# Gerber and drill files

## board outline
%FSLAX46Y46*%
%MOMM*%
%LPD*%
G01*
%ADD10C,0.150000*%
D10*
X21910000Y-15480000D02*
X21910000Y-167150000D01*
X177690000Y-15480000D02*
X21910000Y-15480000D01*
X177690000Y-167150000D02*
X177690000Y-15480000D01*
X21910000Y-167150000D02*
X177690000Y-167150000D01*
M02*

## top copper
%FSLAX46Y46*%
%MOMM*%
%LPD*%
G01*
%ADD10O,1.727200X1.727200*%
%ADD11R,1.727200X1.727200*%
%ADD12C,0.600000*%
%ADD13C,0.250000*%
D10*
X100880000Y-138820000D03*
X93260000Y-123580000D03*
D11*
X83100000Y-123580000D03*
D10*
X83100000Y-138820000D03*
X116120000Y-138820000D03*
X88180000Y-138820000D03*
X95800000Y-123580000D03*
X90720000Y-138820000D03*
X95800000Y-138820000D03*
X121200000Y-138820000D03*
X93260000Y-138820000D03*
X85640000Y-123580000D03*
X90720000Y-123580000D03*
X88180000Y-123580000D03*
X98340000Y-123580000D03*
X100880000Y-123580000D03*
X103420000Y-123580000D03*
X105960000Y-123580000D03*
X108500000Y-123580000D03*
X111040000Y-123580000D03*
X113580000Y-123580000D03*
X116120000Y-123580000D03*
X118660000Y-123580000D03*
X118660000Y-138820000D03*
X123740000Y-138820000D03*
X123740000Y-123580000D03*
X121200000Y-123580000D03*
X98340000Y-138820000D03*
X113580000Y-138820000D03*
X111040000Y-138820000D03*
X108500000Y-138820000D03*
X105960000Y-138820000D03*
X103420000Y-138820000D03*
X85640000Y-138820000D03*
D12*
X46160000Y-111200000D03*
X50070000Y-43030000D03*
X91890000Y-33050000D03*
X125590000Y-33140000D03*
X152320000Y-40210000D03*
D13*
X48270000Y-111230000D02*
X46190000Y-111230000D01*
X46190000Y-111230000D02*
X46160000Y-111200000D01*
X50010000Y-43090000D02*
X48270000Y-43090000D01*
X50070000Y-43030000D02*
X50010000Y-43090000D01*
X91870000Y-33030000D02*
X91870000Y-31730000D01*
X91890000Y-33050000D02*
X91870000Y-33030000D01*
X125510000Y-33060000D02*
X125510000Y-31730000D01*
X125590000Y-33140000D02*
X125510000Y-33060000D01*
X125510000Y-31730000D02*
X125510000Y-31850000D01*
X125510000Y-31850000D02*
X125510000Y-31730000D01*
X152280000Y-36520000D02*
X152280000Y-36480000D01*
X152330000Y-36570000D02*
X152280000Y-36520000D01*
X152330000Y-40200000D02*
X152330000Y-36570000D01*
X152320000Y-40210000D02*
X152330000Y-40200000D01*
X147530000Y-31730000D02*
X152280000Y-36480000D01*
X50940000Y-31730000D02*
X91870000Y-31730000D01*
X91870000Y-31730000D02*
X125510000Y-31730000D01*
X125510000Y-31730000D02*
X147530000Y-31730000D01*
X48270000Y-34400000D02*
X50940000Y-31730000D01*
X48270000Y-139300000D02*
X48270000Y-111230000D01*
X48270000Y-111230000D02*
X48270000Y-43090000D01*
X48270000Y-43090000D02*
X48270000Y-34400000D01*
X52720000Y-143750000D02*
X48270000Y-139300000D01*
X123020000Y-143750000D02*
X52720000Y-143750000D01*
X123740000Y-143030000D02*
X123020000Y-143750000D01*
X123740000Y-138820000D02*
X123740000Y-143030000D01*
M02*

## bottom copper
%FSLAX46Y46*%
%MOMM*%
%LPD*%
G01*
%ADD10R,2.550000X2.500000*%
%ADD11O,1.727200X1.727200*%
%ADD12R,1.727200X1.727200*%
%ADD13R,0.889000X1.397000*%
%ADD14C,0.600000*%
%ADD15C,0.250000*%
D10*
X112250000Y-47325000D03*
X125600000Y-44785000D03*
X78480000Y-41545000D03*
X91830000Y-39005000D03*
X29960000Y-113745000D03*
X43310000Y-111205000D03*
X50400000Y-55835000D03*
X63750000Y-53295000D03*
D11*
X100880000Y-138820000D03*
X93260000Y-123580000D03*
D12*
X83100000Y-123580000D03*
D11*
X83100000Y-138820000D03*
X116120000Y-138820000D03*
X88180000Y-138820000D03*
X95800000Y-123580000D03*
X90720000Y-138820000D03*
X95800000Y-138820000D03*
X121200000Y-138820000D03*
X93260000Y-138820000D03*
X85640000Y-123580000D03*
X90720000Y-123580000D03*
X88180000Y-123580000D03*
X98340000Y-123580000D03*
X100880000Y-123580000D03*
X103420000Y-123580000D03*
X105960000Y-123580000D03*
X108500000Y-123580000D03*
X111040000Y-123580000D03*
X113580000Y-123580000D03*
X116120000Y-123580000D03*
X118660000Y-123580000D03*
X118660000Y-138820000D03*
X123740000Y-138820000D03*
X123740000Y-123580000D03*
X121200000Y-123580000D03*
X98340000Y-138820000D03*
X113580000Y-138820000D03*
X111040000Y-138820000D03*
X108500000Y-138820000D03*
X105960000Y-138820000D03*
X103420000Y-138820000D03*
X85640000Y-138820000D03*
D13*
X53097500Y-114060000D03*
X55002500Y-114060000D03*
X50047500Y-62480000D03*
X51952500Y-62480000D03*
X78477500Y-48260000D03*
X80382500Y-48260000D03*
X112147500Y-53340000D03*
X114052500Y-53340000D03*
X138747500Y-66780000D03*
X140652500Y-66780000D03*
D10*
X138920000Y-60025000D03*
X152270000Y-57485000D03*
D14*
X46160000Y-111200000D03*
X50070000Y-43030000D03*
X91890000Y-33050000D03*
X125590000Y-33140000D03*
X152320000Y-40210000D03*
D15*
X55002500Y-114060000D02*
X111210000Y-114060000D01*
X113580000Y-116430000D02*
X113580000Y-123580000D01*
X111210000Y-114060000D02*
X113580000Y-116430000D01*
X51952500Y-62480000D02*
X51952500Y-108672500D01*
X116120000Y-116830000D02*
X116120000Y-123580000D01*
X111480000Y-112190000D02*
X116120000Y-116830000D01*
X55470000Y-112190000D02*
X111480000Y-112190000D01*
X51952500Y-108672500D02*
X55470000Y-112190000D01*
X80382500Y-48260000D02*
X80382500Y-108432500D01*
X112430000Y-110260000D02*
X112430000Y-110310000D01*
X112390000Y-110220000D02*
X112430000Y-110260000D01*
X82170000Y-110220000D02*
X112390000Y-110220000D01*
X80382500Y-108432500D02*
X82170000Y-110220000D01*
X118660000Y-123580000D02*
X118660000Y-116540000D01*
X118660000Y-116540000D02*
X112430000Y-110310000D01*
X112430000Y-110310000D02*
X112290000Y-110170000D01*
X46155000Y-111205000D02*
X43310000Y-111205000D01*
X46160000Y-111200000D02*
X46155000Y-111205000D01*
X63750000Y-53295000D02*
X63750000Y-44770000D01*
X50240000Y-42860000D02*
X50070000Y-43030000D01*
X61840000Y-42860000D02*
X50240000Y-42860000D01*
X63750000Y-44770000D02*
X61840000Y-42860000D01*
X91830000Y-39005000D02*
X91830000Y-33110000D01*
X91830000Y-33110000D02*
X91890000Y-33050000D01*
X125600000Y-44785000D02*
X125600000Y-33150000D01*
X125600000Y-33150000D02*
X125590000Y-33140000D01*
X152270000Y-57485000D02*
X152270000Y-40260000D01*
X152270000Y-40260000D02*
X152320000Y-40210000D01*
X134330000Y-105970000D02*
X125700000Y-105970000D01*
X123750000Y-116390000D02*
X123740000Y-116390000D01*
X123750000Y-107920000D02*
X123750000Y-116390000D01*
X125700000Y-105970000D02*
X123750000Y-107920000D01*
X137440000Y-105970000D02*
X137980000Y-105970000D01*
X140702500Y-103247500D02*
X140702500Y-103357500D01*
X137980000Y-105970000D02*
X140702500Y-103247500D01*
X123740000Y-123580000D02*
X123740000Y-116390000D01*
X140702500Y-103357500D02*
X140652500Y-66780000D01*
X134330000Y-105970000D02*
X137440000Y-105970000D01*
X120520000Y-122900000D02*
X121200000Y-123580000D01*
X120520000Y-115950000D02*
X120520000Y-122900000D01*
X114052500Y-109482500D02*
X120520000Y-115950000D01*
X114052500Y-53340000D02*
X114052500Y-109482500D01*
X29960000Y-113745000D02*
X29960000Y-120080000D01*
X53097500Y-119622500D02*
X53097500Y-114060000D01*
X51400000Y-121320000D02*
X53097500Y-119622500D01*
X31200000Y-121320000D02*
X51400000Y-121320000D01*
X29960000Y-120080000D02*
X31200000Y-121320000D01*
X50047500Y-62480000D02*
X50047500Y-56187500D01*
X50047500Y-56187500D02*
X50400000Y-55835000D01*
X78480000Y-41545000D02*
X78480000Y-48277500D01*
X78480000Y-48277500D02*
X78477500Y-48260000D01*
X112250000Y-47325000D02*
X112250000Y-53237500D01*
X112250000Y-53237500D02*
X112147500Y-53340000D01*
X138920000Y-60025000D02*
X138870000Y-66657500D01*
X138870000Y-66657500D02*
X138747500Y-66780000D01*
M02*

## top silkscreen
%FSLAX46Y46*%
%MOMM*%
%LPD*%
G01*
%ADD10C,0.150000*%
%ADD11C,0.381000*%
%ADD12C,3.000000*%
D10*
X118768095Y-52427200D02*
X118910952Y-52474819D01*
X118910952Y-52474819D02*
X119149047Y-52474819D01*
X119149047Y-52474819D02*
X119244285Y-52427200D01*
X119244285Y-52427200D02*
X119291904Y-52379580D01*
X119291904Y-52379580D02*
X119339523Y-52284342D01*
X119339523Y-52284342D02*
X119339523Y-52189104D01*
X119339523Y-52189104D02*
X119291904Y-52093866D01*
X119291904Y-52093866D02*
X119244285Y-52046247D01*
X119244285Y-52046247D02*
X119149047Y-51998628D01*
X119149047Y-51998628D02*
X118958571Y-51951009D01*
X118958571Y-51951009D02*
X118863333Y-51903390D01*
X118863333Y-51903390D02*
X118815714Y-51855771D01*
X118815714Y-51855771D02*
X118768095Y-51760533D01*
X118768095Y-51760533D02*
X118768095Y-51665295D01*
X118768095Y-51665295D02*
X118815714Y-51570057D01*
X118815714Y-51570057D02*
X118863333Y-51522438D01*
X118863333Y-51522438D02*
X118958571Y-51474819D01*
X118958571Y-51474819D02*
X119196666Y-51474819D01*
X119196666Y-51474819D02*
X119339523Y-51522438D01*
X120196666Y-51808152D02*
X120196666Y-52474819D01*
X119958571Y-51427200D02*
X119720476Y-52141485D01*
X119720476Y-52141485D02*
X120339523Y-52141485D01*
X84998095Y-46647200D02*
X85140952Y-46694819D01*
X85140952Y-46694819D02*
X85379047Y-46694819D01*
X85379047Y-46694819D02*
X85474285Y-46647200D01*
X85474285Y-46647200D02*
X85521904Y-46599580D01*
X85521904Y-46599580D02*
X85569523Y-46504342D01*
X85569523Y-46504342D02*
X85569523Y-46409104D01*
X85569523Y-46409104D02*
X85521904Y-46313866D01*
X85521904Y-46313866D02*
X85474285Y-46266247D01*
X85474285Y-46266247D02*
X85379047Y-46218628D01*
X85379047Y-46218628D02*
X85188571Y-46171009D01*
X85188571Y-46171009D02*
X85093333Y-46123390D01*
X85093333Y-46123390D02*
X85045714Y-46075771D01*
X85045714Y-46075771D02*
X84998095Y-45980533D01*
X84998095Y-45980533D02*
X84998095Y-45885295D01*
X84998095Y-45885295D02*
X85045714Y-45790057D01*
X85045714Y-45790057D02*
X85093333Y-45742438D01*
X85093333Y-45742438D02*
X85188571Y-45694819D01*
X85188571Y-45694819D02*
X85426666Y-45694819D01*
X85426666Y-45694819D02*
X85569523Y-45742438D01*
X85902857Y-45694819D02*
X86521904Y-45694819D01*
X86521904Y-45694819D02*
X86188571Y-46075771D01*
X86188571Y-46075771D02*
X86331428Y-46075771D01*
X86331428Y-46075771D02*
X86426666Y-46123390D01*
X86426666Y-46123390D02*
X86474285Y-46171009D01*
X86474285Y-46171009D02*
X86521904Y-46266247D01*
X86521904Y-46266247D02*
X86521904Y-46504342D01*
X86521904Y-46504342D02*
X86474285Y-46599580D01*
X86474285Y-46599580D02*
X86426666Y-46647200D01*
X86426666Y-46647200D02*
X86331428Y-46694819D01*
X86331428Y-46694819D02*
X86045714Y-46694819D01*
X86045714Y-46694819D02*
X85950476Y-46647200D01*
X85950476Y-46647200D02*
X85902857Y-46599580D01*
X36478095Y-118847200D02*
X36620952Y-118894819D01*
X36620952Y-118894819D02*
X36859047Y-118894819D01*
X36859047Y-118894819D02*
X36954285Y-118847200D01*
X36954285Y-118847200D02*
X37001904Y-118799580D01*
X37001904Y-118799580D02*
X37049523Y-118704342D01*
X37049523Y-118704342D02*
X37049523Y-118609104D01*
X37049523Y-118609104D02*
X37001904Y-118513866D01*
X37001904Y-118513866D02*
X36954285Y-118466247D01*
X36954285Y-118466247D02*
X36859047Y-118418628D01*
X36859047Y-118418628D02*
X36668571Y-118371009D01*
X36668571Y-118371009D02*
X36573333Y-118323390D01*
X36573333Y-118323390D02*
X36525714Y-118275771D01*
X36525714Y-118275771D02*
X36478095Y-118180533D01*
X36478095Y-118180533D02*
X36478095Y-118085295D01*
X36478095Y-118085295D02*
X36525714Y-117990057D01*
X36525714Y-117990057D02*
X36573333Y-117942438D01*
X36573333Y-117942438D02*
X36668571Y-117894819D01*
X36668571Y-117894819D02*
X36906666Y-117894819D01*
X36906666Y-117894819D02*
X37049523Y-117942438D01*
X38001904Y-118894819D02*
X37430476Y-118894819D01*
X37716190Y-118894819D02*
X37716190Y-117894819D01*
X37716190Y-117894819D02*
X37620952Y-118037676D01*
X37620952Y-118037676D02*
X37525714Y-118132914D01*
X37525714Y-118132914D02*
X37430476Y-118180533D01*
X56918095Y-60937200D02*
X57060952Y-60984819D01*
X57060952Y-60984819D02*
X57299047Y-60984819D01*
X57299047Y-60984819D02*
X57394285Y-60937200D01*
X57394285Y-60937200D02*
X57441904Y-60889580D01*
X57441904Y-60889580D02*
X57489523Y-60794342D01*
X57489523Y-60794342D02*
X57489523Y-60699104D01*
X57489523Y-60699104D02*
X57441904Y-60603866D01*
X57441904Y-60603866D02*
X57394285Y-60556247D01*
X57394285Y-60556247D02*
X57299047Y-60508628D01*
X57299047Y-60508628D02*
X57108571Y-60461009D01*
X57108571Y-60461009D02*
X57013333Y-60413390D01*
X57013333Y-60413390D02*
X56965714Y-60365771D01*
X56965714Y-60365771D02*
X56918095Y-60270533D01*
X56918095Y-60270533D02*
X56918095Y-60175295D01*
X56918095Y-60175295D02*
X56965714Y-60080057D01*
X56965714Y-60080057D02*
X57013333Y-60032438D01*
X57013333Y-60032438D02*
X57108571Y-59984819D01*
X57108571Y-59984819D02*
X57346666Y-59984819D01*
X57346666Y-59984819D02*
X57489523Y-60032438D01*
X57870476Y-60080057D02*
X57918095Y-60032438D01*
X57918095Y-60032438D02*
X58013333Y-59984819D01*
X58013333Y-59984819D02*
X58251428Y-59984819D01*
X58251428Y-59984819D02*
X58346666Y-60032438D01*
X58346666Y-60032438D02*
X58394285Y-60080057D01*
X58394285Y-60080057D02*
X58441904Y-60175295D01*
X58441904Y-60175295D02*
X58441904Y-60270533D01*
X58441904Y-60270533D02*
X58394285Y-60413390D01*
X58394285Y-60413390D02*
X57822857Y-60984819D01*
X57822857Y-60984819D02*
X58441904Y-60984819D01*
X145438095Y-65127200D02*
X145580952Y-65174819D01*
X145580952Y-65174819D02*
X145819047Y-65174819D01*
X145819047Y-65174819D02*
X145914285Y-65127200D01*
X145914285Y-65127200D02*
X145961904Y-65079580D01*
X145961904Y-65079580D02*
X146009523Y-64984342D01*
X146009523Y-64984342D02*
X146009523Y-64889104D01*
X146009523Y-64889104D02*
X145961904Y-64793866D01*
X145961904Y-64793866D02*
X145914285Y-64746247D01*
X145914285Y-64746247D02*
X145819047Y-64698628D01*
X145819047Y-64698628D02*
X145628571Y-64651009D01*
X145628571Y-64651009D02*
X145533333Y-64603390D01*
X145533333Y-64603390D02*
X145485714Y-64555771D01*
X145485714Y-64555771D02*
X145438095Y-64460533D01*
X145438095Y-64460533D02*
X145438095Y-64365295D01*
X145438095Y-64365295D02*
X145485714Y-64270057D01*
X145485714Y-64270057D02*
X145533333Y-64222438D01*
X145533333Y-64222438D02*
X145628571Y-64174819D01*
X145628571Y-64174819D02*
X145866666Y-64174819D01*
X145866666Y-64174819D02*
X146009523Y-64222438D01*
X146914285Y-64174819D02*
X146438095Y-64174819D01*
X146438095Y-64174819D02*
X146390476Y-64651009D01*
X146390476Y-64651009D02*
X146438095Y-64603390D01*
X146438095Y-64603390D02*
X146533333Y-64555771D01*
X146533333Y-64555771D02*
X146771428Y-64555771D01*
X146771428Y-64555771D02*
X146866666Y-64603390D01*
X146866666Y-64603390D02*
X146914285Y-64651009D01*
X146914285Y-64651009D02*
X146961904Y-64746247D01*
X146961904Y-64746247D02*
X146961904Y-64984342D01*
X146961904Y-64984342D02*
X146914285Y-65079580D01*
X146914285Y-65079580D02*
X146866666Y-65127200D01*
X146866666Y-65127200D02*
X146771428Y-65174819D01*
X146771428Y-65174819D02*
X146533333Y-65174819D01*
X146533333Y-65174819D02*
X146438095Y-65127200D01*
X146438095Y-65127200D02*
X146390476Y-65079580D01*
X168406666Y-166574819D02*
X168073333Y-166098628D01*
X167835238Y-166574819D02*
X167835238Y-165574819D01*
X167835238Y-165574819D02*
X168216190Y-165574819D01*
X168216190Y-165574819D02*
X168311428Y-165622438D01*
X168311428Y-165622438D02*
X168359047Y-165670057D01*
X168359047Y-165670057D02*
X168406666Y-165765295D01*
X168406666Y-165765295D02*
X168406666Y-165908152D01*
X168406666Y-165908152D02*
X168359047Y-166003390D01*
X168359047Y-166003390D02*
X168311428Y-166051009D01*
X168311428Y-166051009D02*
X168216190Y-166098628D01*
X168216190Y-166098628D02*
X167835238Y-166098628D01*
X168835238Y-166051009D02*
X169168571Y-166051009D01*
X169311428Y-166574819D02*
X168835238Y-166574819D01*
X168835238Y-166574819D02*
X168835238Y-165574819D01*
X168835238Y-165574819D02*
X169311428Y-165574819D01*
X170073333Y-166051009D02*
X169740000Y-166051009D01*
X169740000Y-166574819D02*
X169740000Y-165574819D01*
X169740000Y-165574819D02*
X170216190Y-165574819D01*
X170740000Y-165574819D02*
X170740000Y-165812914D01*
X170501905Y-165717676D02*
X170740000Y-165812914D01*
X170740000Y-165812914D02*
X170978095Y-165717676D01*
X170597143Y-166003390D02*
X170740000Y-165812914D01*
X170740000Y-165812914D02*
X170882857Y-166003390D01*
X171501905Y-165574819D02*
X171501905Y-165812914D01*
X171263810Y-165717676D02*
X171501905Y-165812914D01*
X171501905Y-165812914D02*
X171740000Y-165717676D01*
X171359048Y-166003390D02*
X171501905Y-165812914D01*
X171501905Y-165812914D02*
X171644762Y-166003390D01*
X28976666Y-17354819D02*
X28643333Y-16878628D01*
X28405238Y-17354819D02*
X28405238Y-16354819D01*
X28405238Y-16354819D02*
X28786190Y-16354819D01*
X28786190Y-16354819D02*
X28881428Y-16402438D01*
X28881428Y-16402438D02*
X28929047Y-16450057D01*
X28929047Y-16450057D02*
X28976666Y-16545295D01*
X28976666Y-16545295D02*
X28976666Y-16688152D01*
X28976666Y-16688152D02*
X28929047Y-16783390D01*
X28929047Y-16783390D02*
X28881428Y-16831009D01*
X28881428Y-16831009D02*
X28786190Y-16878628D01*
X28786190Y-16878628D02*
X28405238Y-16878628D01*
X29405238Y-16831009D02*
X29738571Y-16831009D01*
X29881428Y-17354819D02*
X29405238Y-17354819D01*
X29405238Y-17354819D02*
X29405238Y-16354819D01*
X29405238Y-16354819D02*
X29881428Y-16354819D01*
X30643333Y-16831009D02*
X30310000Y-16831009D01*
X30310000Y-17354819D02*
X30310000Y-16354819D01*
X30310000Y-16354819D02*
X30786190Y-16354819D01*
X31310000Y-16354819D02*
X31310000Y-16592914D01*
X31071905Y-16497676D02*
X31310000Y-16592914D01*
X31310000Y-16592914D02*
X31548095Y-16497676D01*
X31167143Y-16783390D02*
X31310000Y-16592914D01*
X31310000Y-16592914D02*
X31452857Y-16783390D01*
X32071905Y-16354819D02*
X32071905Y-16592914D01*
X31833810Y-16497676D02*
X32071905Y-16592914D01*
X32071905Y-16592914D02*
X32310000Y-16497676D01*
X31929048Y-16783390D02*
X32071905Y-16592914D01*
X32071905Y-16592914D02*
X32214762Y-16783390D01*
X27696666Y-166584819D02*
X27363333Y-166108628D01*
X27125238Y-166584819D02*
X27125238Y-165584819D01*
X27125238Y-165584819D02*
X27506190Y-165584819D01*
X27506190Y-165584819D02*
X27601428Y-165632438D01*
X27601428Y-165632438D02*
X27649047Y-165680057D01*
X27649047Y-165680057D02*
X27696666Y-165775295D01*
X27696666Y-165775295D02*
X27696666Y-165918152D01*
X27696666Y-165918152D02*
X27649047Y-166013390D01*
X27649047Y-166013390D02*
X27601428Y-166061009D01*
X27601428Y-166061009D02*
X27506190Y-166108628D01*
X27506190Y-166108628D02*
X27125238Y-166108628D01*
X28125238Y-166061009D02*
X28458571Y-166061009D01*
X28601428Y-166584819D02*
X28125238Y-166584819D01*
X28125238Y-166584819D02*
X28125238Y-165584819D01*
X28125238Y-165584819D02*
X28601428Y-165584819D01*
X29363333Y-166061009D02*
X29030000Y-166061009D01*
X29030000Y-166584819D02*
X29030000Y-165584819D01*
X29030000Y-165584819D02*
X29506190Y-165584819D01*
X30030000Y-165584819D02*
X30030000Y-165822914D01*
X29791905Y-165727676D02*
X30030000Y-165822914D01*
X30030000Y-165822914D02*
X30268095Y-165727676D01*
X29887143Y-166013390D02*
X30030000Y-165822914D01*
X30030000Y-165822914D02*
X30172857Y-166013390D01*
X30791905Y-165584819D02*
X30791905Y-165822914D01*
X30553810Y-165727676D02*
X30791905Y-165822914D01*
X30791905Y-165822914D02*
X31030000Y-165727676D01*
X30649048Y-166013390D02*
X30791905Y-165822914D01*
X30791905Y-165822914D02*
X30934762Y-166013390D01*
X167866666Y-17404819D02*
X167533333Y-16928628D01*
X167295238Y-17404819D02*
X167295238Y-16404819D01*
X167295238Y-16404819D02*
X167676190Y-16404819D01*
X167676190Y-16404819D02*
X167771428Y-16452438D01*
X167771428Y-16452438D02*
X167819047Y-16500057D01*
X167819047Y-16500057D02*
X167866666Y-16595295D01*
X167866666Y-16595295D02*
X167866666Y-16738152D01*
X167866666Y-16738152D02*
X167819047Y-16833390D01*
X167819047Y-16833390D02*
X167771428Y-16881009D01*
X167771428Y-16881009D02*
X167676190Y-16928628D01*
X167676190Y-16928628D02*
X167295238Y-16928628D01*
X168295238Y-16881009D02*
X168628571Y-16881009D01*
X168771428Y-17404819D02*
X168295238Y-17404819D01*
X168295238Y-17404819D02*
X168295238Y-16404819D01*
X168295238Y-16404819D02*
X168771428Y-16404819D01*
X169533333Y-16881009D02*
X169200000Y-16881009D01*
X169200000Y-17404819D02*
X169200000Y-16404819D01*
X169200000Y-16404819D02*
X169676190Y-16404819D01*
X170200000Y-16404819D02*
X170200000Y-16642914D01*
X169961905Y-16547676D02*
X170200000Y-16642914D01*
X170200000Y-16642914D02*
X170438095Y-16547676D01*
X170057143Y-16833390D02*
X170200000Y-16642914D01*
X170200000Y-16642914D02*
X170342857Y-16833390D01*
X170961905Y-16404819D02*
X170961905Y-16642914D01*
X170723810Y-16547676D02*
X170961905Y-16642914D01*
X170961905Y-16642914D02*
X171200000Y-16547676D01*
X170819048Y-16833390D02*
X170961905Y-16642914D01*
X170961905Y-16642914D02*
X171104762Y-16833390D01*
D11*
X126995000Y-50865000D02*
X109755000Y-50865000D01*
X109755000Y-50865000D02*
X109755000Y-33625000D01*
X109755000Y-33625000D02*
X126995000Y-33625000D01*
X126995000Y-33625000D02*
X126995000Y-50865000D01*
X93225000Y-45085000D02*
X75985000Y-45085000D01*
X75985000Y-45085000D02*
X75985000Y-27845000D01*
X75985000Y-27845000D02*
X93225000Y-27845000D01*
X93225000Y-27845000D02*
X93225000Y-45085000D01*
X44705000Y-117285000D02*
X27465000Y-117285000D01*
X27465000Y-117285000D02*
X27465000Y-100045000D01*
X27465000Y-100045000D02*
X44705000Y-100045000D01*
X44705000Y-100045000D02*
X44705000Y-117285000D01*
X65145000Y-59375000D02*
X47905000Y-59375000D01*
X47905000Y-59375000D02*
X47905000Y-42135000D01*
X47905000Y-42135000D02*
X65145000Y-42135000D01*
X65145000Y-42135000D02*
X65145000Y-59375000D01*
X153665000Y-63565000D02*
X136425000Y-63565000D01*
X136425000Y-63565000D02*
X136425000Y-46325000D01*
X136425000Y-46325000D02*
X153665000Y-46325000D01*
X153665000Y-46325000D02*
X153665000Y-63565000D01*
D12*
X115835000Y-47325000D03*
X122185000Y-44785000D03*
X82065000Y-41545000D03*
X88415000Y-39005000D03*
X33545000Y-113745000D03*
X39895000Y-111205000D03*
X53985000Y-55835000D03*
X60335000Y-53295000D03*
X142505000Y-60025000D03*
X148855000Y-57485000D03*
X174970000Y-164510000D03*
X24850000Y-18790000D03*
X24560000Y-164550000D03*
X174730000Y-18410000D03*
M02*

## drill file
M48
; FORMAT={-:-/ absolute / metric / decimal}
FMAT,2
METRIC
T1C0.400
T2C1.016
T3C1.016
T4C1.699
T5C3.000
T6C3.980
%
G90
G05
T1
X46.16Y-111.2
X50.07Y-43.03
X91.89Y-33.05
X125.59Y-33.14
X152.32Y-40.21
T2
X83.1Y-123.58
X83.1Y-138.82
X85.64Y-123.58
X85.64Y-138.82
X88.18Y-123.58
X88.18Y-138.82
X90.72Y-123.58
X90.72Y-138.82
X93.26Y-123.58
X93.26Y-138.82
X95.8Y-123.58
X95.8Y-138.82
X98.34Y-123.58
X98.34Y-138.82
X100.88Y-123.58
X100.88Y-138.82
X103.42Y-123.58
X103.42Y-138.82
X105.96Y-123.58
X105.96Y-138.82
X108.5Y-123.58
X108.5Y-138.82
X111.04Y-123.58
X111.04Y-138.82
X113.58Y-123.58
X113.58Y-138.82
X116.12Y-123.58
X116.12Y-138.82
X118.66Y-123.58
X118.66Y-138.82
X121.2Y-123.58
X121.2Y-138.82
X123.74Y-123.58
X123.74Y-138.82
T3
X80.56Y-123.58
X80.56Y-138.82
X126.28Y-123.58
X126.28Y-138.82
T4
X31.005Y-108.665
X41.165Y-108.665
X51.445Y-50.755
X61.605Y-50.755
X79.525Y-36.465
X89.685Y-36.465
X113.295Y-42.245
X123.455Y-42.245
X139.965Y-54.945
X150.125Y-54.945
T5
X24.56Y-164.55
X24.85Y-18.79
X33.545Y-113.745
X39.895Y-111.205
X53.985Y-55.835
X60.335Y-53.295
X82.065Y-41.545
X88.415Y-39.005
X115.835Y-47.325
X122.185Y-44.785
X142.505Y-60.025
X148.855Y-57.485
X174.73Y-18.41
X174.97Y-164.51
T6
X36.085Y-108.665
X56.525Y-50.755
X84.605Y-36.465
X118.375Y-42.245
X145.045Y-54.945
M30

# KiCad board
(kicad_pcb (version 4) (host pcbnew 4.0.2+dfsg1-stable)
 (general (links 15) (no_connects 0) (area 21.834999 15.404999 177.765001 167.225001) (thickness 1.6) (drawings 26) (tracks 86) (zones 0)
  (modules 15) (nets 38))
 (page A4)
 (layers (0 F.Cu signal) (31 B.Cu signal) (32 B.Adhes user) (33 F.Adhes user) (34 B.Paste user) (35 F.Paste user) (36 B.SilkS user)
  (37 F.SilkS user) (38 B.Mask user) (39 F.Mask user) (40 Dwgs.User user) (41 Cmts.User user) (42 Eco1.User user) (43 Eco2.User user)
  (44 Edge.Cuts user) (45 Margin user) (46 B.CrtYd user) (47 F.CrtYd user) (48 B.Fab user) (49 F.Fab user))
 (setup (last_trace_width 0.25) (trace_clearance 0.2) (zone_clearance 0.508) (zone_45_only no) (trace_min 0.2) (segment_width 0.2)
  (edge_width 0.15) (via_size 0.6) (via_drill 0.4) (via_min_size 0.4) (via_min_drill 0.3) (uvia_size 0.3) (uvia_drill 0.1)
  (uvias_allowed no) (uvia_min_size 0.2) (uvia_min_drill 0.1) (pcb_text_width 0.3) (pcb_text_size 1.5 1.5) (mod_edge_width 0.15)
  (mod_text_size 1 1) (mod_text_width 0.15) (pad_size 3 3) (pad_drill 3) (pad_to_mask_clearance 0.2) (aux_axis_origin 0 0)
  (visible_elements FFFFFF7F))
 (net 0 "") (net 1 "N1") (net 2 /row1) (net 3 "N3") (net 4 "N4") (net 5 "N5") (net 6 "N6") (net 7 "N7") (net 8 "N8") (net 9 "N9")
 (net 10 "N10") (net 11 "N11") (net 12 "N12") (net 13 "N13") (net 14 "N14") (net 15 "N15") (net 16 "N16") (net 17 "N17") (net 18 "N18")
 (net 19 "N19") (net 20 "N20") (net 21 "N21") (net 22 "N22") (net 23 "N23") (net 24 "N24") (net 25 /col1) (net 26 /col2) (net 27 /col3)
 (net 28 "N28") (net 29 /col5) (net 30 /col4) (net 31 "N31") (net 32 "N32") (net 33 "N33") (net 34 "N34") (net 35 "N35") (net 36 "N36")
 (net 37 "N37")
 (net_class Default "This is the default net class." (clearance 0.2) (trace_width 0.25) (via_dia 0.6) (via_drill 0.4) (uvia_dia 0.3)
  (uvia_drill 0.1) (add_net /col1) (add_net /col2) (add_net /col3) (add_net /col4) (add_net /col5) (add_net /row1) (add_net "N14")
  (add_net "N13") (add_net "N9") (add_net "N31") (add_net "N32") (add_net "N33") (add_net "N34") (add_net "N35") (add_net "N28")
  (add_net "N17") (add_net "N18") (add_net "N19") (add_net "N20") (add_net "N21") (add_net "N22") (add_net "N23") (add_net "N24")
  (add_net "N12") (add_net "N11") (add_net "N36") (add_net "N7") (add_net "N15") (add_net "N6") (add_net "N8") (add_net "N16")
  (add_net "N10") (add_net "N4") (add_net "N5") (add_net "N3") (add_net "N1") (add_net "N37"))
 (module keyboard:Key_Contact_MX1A (layer F.Cu) (at 118.43 42.29)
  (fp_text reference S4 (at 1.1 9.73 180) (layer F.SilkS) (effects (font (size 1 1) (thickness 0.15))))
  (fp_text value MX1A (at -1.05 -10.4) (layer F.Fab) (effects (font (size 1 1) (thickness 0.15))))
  (fp_line (start 8.565 8.575) (end -8.675 8.575) (layer F.SilkS) (width 0.381))
  (fp_line (start -8.675 8.575) (end -8.675 -8.665) (layer F.SilkS) (width 0.381))
  (fp_line (start -8.675 -8.665) (end 8.565 -8.665) (layer F.SilkS) (width 0.381))
  (fp_line (start 8.565 -8.665) (end 8.565 8.575) (layer F.SilkS) (width 0.381))
  (pad "" np_thru_hole circle (at -0.055 -0.045 180) (size 3.98018 3.98018) (drill 3.98018) (layers *.Cu *.Mask))
  (pad "" np_thru_hole circle (at -2.595 5.035 180) (size 3 3) (drill 3) (layers *.Cu *.Mask F.SilkS))
  (pad "" np_thru_hole circle (at 3.755 2.495 180) (size 3 3) (drill 3) (layers *.Cu *.Mask F.SilkS))
  (pad "" np_thru_hole circle (at 5.025 -0.045 180) (size 1.69926 1.69926) (drill 1.69926) (layers *.Cu *.Mask))
  (pad "" np_thru_hole circle (at -5.135 -0.045 180) (size 1.69926 1.69926) (drill 1.69926) (layers *.Cu *.Mask))
  (pad 2 smd rect (at -6.18 5.035) (size 2.55 2.5) (layers B.Cu B.Paste B.Mask) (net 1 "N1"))
  (pad 1 smd rect (at 7.17 2.495 180) (size 2.55 2.5) (layers B.Cu B.Paste B.Mask) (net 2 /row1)))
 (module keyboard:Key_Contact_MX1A (layer F.Cu) (at 84.66 36.51)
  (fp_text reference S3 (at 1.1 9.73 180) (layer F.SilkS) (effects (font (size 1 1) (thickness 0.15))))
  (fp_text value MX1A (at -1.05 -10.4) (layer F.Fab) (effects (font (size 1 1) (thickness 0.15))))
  (fp_line (start 8.565 8.575) (end -8.675 8.575) (layer F.SilkS) (width 0.381))
  (fp_line (start -8.675 8.575) (end -8.675 -8.665) (layer F.SilkS) (width 0.381))
  (fp_line (start -8.675 -8.665) (end 8.565 -8.665) (layer F.SilkS) (width 0.381))
  (fp_line (start 8.565 -8.665) (end 8.565 8.575) (layer F.SilkS) (width 0.381))
  (pad "" np_thru_hole circle (at -0.055 -0.045 180) (size 3.98018 3.98018) (drill 3.98018) (layers *.Cu *.Mask))
  (pad "" np_thru_hole circle (at -2.595 5.035 180) (size 3 3) (drill 3) (layers *.Cu *.Mask F.SilkS))
  (pad "" np_thru_hole circle (at 3.755 2.495 180) (size 3 3) (drill 3) (layers *.Cu *.Mask F.SilkS))
  (pad "" np_thru_hole circle (at 5.025 -0.045 180) (size 1.69926 1.69926) (drill 1.69926) (layers *.Cu *.Mask))
  (pad "" np_thru_hole circle (at -5.135 -0.045 180) (size 1.69926 1.69926) (drill 1.69926) (layers *.Cu *.Mask))
  (pad 2 smd rect (at -6.18 5.035) (size 2.55 2.5) (layers B.Cu B.Paste B.Mask) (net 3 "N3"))
  (pad 1 smd rect (at 7.17 2.495 180) (size 2.55 2.5) (layers B.Cu B.Paste B.Mask) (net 2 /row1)))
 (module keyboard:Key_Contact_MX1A (layer F.Cu) (at 36.14 108.71)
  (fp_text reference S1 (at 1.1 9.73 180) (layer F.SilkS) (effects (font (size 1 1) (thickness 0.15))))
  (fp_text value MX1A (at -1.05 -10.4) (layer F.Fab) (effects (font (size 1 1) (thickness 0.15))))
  (fp_line (start 8.565 8.575) (end -8.675 8.575) (layer F.SilkS) (width 0.381))
  (fp_line (start -8.675 8.575) (end -8.675 -8.665) (layer F.SilkS) (width 0.381))
  (fp_line (start -8.675 -8.665) (end 8.565 -8.665) (layer F.SilkS) (width 0.381))
  (fp_line (start 8.565 -8.665) (end 8.565 8.575) (layer F.SilkS) (width 0.381))
  (pad "" np_thru_hole circle (at -0.055 -0.045 180) (size 3.98018 3.98018) (drill 3.98018) (layers *.Cu *.Mask))
  (pad "" np_thru_hole circle (at -2.595 5.035 180) (size 3 3) (drill 3) (layers *.Cu *.Mask F.SilkS))
  (pad "" np_thru_hole circle (at 3.755 2.495 180) (size 3 3) (drill 3) (layers *.Cu *.Mask F.SilkS))
  (pad "" np_thru_hole circle (at 5.025 -0.045 180) (size 1.69926 1.69926) (drill 1.69926) (layers *.Cu *.Mask))
  (pad "" np_thru_hole circle (at -5.135 -0.045 180) (size 1.69926 1.69926) (drill 1.69926) (layers *.Cu *.Mask))
  (pad 2 smd rect (at -6.18 5.035) (size 2.55 2.5) (layers B.Cu B.Paste B.Mask) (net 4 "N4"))
  (pad 1 smd rect (at 7.17 2.495 180) (size 2.55 2.5) (layers B.Cu B.Paste B.Mask) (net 2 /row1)))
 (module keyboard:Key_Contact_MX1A (layer F.Cu) (at 56.58 50.8)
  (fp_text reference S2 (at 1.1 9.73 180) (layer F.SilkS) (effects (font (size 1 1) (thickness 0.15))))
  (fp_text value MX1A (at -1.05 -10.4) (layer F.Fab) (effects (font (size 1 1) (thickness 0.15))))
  (fp_line (start 8.565 8.575) (end -8.675 8.575) (layer F.SilkS) (width 0.381))
  (fp_line (start -8.675 8.575) (end -8.675 -8.665) (layer F.SilkS) (width 0.381))
  (fp_line (start -8.675 -8.665) (end 8.565 -8.665) (layer F.SilkS) (width 0.381))
  (fp_line (start 8.565 -8.665) (end 8.565 8.575) (layer F.SilkS) (width 0.381))
  (pad "" np_thru_hole circle (at -0.055 -0.045 180) (size 3.98018 3.98018) (drill 3.98018) (layers *.Cu *.Mask))
  (pad "" np_thru_hole circle (at -2.595 5.035 180) (size 3 3) (drill 3) (layers *.Cu *.Mask F.SilkS))
  (pad "" np_thru_hole circle (at 3.755 2.495 180) (size 3 3) (drill 3) (layers *.Cu *.Mask F.SilkS))
  (pad "" np_thru_hole circle (at 5.025 -0.045 180) (size 1.69926 1.69926) (drill 1.69926) (layers *.Cu *.Mask))
  (pad "" np_thru_hole circle (at -5.135 -0.045 180) (size 1.69926 1.69926) (drill 1.69926) (layers *.Cu *.Mask))
  (pad 2 smd rect (at -6.18 5.035) (size 2.55 2.5) (layers B.Cu B.Paste B.Mask) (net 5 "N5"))
  (pad 1 smd rect (at 7.17 2.495 180) (size 2.55 2.5) (layers B.Cu B.Paste B.Mask) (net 2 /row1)))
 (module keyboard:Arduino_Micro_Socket (layer B.Cu) (at 127.66 140.2 180)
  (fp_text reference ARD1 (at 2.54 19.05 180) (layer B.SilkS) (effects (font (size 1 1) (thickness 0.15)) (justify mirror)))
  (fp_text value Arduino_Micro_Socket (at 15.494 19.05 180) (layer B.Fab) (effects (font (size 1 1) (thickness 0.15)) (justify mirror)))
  (pad "" np_thru_hole circle (at 47.1 16.62 180) (size 1.016 1.016) (drill 1.016) (layers *.Cu *.Mask))
  (pad "" np_thru_hole circle (at 1.38 16.62 180) (size 1.016 1.016) (drill 1.016) (layers *.Cu *.Mask))
  (pad "" np_thru_hole circle (at 47.1 1.38 180) (size 1.016 1.016) (drill 1.016) (layers *.Cu *.Mask))
  (pad "" thru_hole oval (at 26.78 1.38 180) (size 1.7272 1.7272) (drill 1.016) (layers *.Cu *.Mask))
  (pad RST2 thru_hole oval (at 34.4 16.62 180) (size 1.7272 1.7272) (drill 1.016) (layers *.Cu *.Mask) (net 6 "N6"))
  (pad MOSI thru_hole rect (at 44.56 16.62 180) (size 1.7272 1.7272) (drill 1.016) (layers *.Cu *.Mask) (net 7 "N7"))
  (pad SCK thru_hole oval (at 44.56 1.38 180) (size 1.7272 1.7272) (drill 1.016) (layers *.Cu *.Mask) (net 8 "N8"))
  (pad A0 thru_hole oval (at 11.54 1.38 180) (size 1.7272 1.7272) (drill 1.016) (layers *.Cu *.Mask) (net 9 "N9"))
  (pad VIN thru_hole oval (at 39.48 1.38 180) (size 1.7272 1.7272) (drill 1.016) (layers *.Cu *.Mask) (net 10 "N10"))
  (pad GND2 thru_hole oval (at 31.86 16.62 180) (size 1.7272 1.7272) (drill 1.016) (layers *.Cu *.Mask) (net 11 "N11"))
  (pad GND1 thru_hole oval (at 36.94 1.38 180) (size 1.7272 1.7272) (drill 1.016) (layers *.Cu *.Mask) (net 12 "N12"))
  (pad 5V thru_hole oval (at 31.86 1.38 180) (size 1.7272 1.7272) (drill 1.016) (layers *.Cu *.Mask) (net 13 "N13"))
  (pad 3.3V thru_hole oval (at 6.46 1.38 180) (size 1.7272 1.7272) (drill 1.016) (layers *.Cu *.Mask) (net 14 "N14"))
  (pad RST1 thru_hole oval (at 34.4 1.38 180) (size 1.7272 1.7272) (drill 1.016) (layers *.Cu *.Mask) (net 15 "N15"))
  (pad SS thru_hole oval (at 42.02 16.62 180) (size 1.7272 1.7272) (drill 1.016) (layers *.Cu *.Mask) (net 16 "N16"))
  (pad D0 thru_hole oval (at 36.94 16.62 180) (size 1.7272 1.7272) (drill 1.016) (layers *.Cu *.Mask) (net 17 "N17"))
  (pad D1 thru_hole oval (at 39.48 16.62 180) (size 1.7272 1.7272) (drill 1.016) (layers *.Cu *.Mask) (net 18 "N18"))
  (pad D2 thru_hole oval (at 29.32 16.62 180) (size 1.7272 1.7272) (drill 1.016) (layers *.Cu *.Mask) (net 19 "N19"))
  (pad D3 thru_hole oval (at 26.78 16.62 180) (size 1.7272 1.7272) (drill 1.016) (layers *.Cu *.Mask) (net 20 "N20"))
  (pad D4 thru_hole oval (at 24.24 16.62 180) (size 1.7272 1.7272) (drill 1.016) (layers *.Cu *.Mask) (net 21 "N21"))
  (pad D5 thru_hole oval (at 21.7 16.62 180) (size 1.7272 1.7272) (drill 1.016) (layers *.Cu *.Mask) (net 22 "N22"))
  (pad D6 thru_hole oval (at 19.16 16.62 180) (size 1.7272 1.7272) (drill 1.016) (layers *.Cu *.Mask) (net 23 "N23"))
  (pad D7 thru_hole oval (at 16.62 16.62 180) (size 1.7272 1.7272) (drill 1.016) (layers *.Cu *.Mask) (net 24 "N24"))
  (pad D8 thru_hole oval (at 14.08 16.62 180) (size 1.7272 1.7272) (drill 1.016) (layers *.Cu *.Mask) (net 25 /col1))
  (pad D9 thru_hole oval (at 11.54 16.62 180) (size 1.7272 1.7272) (drill 1.016) (layers *.Cu *.Mask) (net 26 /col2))
  (pad D10 thru_hole oval (at 9 16.62 180) (size 1.7272 1.7272) (drill 1.016) (layers *.Cu *.Mask) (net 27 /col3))
  (pad "" np_thru_hole circle (at 1.38 1.38 180) (size 1.016 1.016) (drill 1.016) (layers *.Cu *.Mask))
  (pad AREF thru_hole oval (at 9 1.38 180) (size 1.7272 1.7272) (drill 1.016) (layers *.Cu *.Mask) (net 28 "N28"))
  (pad D13 thru_hole oval (at 3.92 1.38 180) (size 1.7272 1.7272) (drill 1.016) (layers *.Cu *.Mask) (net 2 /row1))
  (pad D12 thru_hole oval (at 3.92 16.62 180) (size 1.7272 1.7272) (drill 1.016) (layers *.Cu *.Mask) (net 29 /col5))
  (pad D11 thru_hole oval (at 6.46 16.62 180) (size 1.7272 1.7272) (drill 1.016) (layers *.Cu *.Mask) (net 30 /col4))
  (pad "" thru_hole oval (at 29.32 1.38 180) (size 1.7272 1.7272) (drill 1.016) (layers *.Cu *.Mask))
  (pad A1 thru_hole oval (at 14.08 1.38 180) (size 1.7272 1.7272) (drill 1.016) (layers *.Cu *.Mask) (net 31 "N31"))
  (pad A2 thru_hole oval (at 16.62 1.38 180) (size 1.7272 1.7272) (drill 1.016) (layers *.Cu *.Mask) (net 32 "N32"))
  (pad A3 thru_hole oval (at 19.16 1.38 180) (size 1.7272 1.7272) (drill 1.016) (layers *.Cu *.Mask) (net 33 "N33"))
  (pad A4 thru_hole oval (at 21.7 1.38 180) (size 1.7272 1.7272) (drill 1.016) (layers *.Cu *.Mask) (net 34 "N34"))
  (pad A5 thru_hole oval (at 24.24 1.38 180) (size 1.7272 1.7272) (drill 1.016) (layers *.Cu *.Mask) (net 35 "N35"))
  (pad MISO thru_hole oval (at 42.02 1.38 180) (size 1.7272 1.7272) (drill 1.016) (layers *.Cu *.Mask) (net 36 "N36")))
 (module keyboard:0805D (layer B.Cu) (at 54.05 114.06)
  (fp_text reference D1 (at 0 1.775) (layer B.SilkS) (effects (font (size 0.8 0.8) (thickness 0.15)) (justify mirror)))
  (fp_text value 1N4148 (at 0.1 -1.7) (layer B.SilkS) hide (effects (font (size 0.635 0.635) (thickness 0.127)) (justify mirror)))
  (pad 1 smd rect (at -0.9525 0) (size 0.889 1.397) (layers B.Cu B.Paste B.Mask) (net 4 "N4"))
  (pad 2 smd rect (at 0.9525 0) (size 0.889 1.397) (layers B.Cu B.Paste B.Mask) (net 25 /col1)))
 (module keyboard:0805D (layer B.Cu) (at 51 62.48)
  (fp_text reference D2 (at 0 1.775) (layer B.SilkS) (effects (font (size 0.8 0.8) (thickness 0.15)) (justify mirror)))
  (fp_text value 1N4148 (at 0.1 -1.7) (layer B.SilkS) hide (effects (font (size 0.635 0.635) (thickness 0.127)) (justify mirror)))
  (pad 1 smd rect (at -0.9525 0) (size 0.889 1.397) (layers B.Cu B.Paste B.Mask) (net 5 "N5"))
  (pad 2 smd rect (at 0.9525 0) (size 0.889 1.397) (layers B.Cu B.Paste B.Mask) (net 26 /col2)))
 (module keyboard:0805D (layer B.Cu) (at 79.43 48.26)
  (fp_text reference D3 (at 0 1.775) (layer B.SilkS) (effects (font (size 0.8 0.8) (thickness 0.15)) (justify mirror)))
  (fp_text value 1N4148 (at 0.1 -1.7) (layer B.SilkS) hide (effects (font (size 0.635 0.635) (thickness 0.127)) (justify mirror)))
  (pad 1 smd rect (at -0.9525 0) (size 0.889 1.397) (layers B.Cu B.Paste B.Mask) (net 3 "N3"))
  (pad 2 smd rect (at 0.9525 0) (size 0.889 1.397) (layers B.Cu B.Paste B.Mask) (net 27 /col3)))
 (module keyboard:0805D (layer B.Cu) (at 113.1 53.34)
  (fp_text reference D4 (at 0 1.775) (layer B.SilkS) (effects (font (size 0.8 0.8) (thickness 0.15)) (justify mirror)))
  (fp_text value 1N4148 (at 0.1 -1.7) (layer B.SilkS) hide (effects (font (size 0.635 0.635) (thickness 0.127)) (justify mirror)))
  (pad 1 smd rect (at -0.9525 0) (size 0.889 1.397) (layers B.Cu B.Paste B.Mask) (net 1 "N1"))
  (pad 2 smd rect (at 0.9525 0) (size 0.889 1.397) (layers B.Cu B.Paste B.Mask) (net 30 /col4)))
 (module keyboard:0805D (layer B.Cu) (at 139.7 66.78)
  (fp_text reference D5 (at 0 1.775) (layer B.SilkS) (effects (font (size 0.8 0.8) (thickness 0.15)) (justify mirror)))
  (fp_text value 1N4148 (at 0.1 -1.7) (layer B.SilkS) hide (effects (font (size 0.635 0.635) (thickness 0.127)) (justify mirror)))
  (pad 1 smd rect (at -0.9525 0) (size 0.889 1.397) (layers B.Cu B.Paste B.Mask) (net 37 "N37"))
  (pad 2 smd rect (at 0.9525 0) (size 0.889 1.397) (layers B.Cu B.Paste B.Mask) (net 29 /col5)))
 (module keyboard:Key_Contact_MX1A (layer F.Cu) (at 145.1 54.99)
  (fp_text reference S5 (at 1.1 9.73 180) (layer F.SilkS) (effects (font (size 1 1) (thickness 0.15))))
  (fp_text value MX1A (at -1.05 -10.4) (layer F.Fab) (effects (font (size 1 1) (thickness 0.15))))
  (fp_line (start 8.565 8.575) (end -8.675 8.575) (layer F.SilkS) (width 0.381))
  (fp_line (start -8.675 8.575) (end -8.675 -8.665) (layer F.SilkS) (width 0.381))
  (fp_line (start -8.675 -8.665) (end 8.565 -8.665) (layer F.SilkS) (width 0.381))
  (fp_line (start 8.565 -8.665) (end 8.565 8.575) (layer F.SilkS) (width 0.381))
  (pad "" np_thru_hole circle (at -0.055 -0.045 180) (size 3.98018 3.98018) (drill 3.98018) (layers *.Cu *.Mask))
  (pad "" np_thru_hole circle (at -2.595 5.035 180) (size 3 3) (drill 3) (layers *.Cu *.Mask F.SilkS))
  (pad "" np_thru_hole circle (at 3.755 2.495 180) (size 3 3) (drill 3) (layers *.Cu *.Mask F.SilkS))
  (pad "" np_thru_hole circle (at 5.025 -0.045 180) (size 1.69926 1.69926) (drill 1.69926) (layers *.Cu *.Mask))
  (pad "" np_thru_hole circle (at -5.135 -0.045 180) (size 1.69926 1.69926) (drill 1.69926) (layers *.Cu *.Mask))
  (pad 2 smd rect (at -6.18 5.035) (size 2.55 2.5) (layers B.Cu B.Paste B.Mask) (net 37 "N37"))
  (pad 1 smd rect (at 7.17 2.495 180) (size 2.55 2.5) (layers B.Cu B.Paste B.Mask) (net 2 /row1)))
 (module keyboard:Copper (layer F.Cu) (at 174.99 164.48)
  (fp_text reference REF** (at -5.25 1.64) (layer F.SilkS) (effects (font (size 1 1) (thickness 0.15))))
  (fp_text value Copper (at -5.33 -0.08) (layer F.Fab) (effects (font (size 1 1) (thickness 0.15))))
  (pad "" np_thru_hole circle (at -0.02 0.03) (size 3 3) (drill 3) (layers *.Cu *.Mask F.SilkS)))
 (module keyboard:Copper (layer F.Cu) (at 24.87 18.76)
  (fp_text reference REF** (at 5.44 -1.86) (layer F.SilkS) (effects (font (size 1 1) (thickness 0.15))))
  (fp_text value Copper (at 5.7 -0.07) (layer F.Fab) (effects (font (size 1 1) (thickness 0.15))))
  (pad "" np_thru_hole circle (at -0.02 0.03) (size 3 3) (drill 3) (layers *.Cu *.Mask F.SilkS)))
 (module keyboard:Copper (layer F.Cu) (at 24.58 164.52)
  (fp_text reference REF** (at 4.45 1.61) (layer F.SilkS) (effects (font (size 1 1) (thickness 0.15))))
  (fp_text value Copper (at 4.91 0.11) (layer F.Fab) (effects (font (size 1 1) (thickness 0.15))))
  (pad "" np_thru_hole circle (at -0.02 0.03) (size 3 3) (drill 3) (layers *.Cu *.Mask F.SilkS)))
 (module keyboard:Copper (layer F.Cu) (at 174.75 18.38)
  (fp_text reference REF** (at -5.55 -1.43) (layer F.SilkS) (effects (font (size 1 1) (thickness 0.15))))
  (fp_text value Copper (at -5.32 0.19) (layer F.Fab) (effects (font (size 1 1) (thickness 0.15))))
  (pad "" np_thru_hole circle (at -0.02 0.03) (size 3 3) (drill 3) (layers *.Cu *.Mask F.SilkS)))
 (gr_line (start 21.91 15.48) (end 21.91 167.15) (angle 90) (layer Edge.Cuts) (width 0.15))
 (gr_line (start 177.69 15.48) (end 21.91 15.48) (angle 90) (layer Edge.Cuts) (width 0.15))
 (gr_line (start 177.69 167.15) (end 177.69 15.48) (angle 90) (layer Edge.Cuts) (width 0.15))
 (gr_line (start 21.91 167.15) (end 177.69 167.15) (angle 90) (layer Edge.Cuts) (width 0.15))
 (segment (start 55.0025 114.06) (end 111.21 114.06) (width 0.25) (layer B.Cu) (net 25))
 (segment (start 113.58 116.43) (end 113.58 123.58) (width 0.25) (layer B.Cu) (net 25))
 (segment (start 111.21 114.06) (end 113.58 116.43) (width 0.25) (layer B.Cu) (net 25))
 (segment (start 51.9525 62.48) (end 51.9525 108.6725) (width 0.25) (layer B.Cu) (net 26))
 (segment (start 116.12 116.83) (end 116.12 123.58) (width 0.25) (layer B.Cu) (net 26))
 (segment (start 111.48 112.19) (end 116.12 116.83) (width 0.25) (layer B.Cu) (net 26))
 (segment (start 55.47 112.19) (end 111.48 112.19) (width 0.25) (layer B.Cu) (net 26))
 (segment (start 51.9525 108.6725) (end 55.47 112.19) (width 0.25) (layer B.Cu) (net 26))
 (segment (start 80.3825 48.26) (end 80.3825 108.4325) (width 0.25) (layer B.Cu) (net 27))
 (segment (start 112.43 110.26) (end 112.43 110.31) (width 0.25) (layer B.Cu) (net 27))
 (segment (start 112.39 110.22) (end 112.43 110.26) (width 0.25) (layer B.Cu) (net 27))
 (segment (start 82.17 110.22) (end 112.39 110.22) (width 0.25) (layer B.Cu) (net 27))
 (segment (start 80.3825 108.4325) (end 82.17 110.22) (width 0.25) (layer B.Cu) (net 27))
 (segment (start 118.66 123.58) (end 118.66 116.54) (width 0.25) (layer B.Cu) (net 27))
 (segment (start 118.66 116.54) (end 112.43 110.31) (width 0.25) (layer B.Cu) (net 27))
 (segment (start 112.43 110.31) (end 112.29 110.17) (width 0.25) (layer B.Cu) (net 27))
 (segment (start 48.27 111.23) (end 46.19 111.23) (width 0.25) (layer F.Cu) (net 2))
 (segment (start 46.155 111.205) (end 43.31 111.205) (width 0.25) (layer B.Cu) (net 2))
 (segment (start 46.16 111.2) (end 46.155 111.205) (width 0.25) (layer B.Cu) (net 2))
 (via (at 46.16 111.2) (size 0.6) (drill 0.4) (layers F.Cu B.Cu) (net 2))
 (segment (start 46.19 111.23) (end 46.16 111.2) (width 0.25) (layer F.Cu) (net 2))
 (segment (start 63.75 53.295) (end 63.75 44.77) (width 0.25) (layer B.Cu) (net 2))
 (segment (start 50.01 43.09) (end 48.27 43.09) (width 0.25) (layer F.Cu) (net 2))
 (segment (start 50.07 43.03) (end 50.01 43.09) (width 0.25) (layer F.Cu) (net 2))
 (via (at 50.07 43.03) (size 0.6) (drill 0.4) (layers F.Cu B.Cu) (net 2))
 (segment (start 50.24 42.86) (end 50.07 43.03) (width 0.25) (layer B.Cu) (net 2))
 (segment (start 61.84 42.86) (end 50.24 42.86) (width 0.25) (layer B.Cu) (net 2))
 (segment (start 63.75 44.77) (end 61.84 42.86) (width 0.25) (layer B.Cu) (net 2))
 (segment (start 91.83 39.005) (end 91.83 33.11) (width 0.25) (layer B.Cu) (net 2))
 (segment (start 91.87 33.03) (end 91.87 31.73) (width 0.25) (layer F.Cu) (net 2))
 (segment (start 91.89 33.05) (end 91.87 33.03) (width 0.25) (layer F.Cu) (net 2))
 (via (at 91.89 33.05) (size 0.6) (drill 0.4) (layers F.Cu B.Cu) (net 2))
 (segment (start 91.83 33.11) (end 91.89 33.05) (width 0.25) (layer B.Cu) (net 2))
 (segment (start 125.6 44.785) (end 125.6 33.15) (width 0.25) (layer B.Cu) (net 2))
 (segment (start 125.51 33.06) (end 125.51 31.73) (width 0.25) (layer F.Cu) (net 2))
 (segment (start 125.59 33.14) (end 125.51 33.06) (width 0.25) (layer F.Cu) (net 2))
 (via (at 125.59 33.14) (size 0.6) (drill 0.4) (layers F.Cu B.Cu) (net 2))
 (segment (start 125.6 33.15) (end 125.59 33.14) (width 0.25) (layer B.Cu) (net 2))
 (segment (start 125.51 31.73) (end 125.51 31.85) (width 0.25) (layer F.Cu) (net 2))
 (segment (start 125.51 31.85) (end 125.51 31.73) (width 0.25) (layer F.Cu) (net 2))
 (segment (start 152.27 57.485) (end 152.27 40.26) (width 0.25) (layer B.Cu) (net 2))
 (segment (start 152.28 36.52) (end 152.28 36.48) (width 0.25) (layer F.Cu) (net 2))
 (segment (start 152.33 36.57) (end 152.28 36.52) (width 0.25) (layer F.Cu) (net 2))
 (segment (start 152.33 40.2) (end 152.33 36.57) (width 0.25) (layer F.Cu) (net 2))
 (segment (start 152.32 40.21) (end 152.33 40.2) (width 0.25) (layer F.Cu) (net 2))
 (via (at 152.32 40.21) (size 0.6) (drill 0.4) (layers F.Cu B.Cu) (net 2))
 (segment (start 152.27 40.26) (end 152.32 40.21) (width 0.25) (layer B.Cu) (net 2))
 (segment (start 147.53 31.73) (end 152.28 36.48) (width 0.25) (layer F.Cu) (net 2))
 (segment (start 50.94 31.73) (end 91.87 31.73) (width 0.25) (layer F.Cu) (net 2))
 (segment (start 91.87 31.73) (end 125.51 31.73) (width 0.25) (layer F.Cu) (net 2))
 (segment (start 125.51 31.73) (end 147.53 31.73) (width 0.25) (layer F.Cu) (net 2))
 (segment (start 48.27 34.4) (end 50.94 31.73) (width 0.25) (layer F.Cu) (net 2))
 (segment (start 48.27 139.3) (end 48.27 111.23) (width 0.25) (layer F.Cu) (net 2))
 (segment (start 48.27 111.23) (end 48.27 43.09) (width 0.25) (layer F.Cu) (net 2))
 (segment (start 48.27 43.09) (end 48.27 34.4) (width 0.25) (layer F.Cu) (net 2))
 (segment (start 52.72 143.75) (end 48.27 139.3) (width 0.25) (layer F.Cu) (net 2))
 (segment (start 123.02 143.75) (end 52.72 143.75) (width 0.25) (layer F.Cu) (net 2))
 (segment (start 123.74 143.03) (end 123.02 143.75) (width 0.25) (layer F.Cu) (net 2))
 (segment (start 123.74 138.82) (end 123.74 143.03) (width 0.25) (layer F.Cu) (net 2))
 (segment (start 134.33 105.97) (end 125.7 105.97) (width 0.25) (layer B.Cu) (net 29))
 (segment (start 123.75 116.39) (end 123.74 116.39) (width 0.25) (layer B.Cu) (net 29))
 (segment (start 123.75 107.92) (end 123.75 116.39) (width 0.25) (layer B.Cu) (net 29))
 (segment (start 125.7 105.97) (end 123.75 107.92) (width 0.25) (layer B.Cu) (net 29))
 (segment (start 137.44 105.97) (end 137.98 105.97) (width 0.25) (layer B.Cu) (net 29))
 (segment (start 140.7025 103.2475) (end 140.7025 103.3575) (width 0.25) (layer B.Cu) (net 29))
 (segment (start 137.98 105.97) (end 140.7025 103.2475) (width 0.25) (layer B.Cu) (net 29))
 (segment (start 123.74 123.58) (end 123.74 116.39) (width 0.25) (layer B.Cu) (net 29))
 (segment (start 140.7025 103.3575) (end 140.6525 66.78) (width 0.25) (layer B.Cu) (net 29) (status 20))
 (segment (start 134.33 105.97) (end 137.44 105.97) (width 0.25) (layer B.Cu) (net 29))
 (segment (start 120.52 122.9) (end 121.2 123.58) (width 0.25) (layer B.Cu) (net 30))
 (segment (start 120.52 115.95) (end 120.52 122.9) (width 0.25) (layer B.Cu) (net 30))
 (segment (start 114.0525 109.4825) (end 120.52 115.95) (width 0.25) (layer B.Cu) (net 30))
 (segment (start 114.0525 53.34) (end 114.0525 109.4825) (width 0.25) (layer B.Cu) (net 30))
 (segment (start 29.96 113.745) (end 29.96 120.08) (width 0.25) (layer B.Cu) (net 4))
 (segment (start 53.0975 119.6225) (end 53.0975 114.06) (width 0.25) (layer B.Cu) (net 4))
 (segment (start 51.4 121.32) (end 53.0975 119.6225) (width 0.25) (layer B.Cu) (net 4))
 (segment (start 31.2 121.32) (end 51.4 121.32) (width 0.25) (layer B.Cu) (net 4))
 (segment (start 29.96 120.08) (end 31.2 121.32) (width 0.25) (layer B.Cu) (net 4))
 (segment (start 50.0475 62.48) (end 50.0475 56.1875) (width 0.25) (layer B.Cu) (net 5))
 (segment (start 50.0475 56.1875) (end 50.4 55.835) (width 0.25) (layer B.Cu) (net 5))
 (segment (start 78.48 41.545) (end 78.48 48.2775) (width 0.25) (layer B.Cu) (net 3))
 (segment (start 78.48 48.2775) (end 78.4775 48.26) (width 0.25) (layer B.Cu) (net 3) (status 20))
 (segment (start 112.25 47.325) (end 112.25 53.2375) (width 0.25) (layer B.Cu) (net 1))
 (segment (start 112.25 53.2375) (end 112.1475 53.34) (width 0.25) (layer B.Cu) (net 1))
 (segment (start 138.92 60.025) (end 138.87 66.6575) (width 0.25) (layer B.Cu) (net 37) (status 20))
 (segment (start 138.87 66.6575) (end 138.7475 66.78) (width 0.25) (layer B.Cu) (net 37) (status 30)))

